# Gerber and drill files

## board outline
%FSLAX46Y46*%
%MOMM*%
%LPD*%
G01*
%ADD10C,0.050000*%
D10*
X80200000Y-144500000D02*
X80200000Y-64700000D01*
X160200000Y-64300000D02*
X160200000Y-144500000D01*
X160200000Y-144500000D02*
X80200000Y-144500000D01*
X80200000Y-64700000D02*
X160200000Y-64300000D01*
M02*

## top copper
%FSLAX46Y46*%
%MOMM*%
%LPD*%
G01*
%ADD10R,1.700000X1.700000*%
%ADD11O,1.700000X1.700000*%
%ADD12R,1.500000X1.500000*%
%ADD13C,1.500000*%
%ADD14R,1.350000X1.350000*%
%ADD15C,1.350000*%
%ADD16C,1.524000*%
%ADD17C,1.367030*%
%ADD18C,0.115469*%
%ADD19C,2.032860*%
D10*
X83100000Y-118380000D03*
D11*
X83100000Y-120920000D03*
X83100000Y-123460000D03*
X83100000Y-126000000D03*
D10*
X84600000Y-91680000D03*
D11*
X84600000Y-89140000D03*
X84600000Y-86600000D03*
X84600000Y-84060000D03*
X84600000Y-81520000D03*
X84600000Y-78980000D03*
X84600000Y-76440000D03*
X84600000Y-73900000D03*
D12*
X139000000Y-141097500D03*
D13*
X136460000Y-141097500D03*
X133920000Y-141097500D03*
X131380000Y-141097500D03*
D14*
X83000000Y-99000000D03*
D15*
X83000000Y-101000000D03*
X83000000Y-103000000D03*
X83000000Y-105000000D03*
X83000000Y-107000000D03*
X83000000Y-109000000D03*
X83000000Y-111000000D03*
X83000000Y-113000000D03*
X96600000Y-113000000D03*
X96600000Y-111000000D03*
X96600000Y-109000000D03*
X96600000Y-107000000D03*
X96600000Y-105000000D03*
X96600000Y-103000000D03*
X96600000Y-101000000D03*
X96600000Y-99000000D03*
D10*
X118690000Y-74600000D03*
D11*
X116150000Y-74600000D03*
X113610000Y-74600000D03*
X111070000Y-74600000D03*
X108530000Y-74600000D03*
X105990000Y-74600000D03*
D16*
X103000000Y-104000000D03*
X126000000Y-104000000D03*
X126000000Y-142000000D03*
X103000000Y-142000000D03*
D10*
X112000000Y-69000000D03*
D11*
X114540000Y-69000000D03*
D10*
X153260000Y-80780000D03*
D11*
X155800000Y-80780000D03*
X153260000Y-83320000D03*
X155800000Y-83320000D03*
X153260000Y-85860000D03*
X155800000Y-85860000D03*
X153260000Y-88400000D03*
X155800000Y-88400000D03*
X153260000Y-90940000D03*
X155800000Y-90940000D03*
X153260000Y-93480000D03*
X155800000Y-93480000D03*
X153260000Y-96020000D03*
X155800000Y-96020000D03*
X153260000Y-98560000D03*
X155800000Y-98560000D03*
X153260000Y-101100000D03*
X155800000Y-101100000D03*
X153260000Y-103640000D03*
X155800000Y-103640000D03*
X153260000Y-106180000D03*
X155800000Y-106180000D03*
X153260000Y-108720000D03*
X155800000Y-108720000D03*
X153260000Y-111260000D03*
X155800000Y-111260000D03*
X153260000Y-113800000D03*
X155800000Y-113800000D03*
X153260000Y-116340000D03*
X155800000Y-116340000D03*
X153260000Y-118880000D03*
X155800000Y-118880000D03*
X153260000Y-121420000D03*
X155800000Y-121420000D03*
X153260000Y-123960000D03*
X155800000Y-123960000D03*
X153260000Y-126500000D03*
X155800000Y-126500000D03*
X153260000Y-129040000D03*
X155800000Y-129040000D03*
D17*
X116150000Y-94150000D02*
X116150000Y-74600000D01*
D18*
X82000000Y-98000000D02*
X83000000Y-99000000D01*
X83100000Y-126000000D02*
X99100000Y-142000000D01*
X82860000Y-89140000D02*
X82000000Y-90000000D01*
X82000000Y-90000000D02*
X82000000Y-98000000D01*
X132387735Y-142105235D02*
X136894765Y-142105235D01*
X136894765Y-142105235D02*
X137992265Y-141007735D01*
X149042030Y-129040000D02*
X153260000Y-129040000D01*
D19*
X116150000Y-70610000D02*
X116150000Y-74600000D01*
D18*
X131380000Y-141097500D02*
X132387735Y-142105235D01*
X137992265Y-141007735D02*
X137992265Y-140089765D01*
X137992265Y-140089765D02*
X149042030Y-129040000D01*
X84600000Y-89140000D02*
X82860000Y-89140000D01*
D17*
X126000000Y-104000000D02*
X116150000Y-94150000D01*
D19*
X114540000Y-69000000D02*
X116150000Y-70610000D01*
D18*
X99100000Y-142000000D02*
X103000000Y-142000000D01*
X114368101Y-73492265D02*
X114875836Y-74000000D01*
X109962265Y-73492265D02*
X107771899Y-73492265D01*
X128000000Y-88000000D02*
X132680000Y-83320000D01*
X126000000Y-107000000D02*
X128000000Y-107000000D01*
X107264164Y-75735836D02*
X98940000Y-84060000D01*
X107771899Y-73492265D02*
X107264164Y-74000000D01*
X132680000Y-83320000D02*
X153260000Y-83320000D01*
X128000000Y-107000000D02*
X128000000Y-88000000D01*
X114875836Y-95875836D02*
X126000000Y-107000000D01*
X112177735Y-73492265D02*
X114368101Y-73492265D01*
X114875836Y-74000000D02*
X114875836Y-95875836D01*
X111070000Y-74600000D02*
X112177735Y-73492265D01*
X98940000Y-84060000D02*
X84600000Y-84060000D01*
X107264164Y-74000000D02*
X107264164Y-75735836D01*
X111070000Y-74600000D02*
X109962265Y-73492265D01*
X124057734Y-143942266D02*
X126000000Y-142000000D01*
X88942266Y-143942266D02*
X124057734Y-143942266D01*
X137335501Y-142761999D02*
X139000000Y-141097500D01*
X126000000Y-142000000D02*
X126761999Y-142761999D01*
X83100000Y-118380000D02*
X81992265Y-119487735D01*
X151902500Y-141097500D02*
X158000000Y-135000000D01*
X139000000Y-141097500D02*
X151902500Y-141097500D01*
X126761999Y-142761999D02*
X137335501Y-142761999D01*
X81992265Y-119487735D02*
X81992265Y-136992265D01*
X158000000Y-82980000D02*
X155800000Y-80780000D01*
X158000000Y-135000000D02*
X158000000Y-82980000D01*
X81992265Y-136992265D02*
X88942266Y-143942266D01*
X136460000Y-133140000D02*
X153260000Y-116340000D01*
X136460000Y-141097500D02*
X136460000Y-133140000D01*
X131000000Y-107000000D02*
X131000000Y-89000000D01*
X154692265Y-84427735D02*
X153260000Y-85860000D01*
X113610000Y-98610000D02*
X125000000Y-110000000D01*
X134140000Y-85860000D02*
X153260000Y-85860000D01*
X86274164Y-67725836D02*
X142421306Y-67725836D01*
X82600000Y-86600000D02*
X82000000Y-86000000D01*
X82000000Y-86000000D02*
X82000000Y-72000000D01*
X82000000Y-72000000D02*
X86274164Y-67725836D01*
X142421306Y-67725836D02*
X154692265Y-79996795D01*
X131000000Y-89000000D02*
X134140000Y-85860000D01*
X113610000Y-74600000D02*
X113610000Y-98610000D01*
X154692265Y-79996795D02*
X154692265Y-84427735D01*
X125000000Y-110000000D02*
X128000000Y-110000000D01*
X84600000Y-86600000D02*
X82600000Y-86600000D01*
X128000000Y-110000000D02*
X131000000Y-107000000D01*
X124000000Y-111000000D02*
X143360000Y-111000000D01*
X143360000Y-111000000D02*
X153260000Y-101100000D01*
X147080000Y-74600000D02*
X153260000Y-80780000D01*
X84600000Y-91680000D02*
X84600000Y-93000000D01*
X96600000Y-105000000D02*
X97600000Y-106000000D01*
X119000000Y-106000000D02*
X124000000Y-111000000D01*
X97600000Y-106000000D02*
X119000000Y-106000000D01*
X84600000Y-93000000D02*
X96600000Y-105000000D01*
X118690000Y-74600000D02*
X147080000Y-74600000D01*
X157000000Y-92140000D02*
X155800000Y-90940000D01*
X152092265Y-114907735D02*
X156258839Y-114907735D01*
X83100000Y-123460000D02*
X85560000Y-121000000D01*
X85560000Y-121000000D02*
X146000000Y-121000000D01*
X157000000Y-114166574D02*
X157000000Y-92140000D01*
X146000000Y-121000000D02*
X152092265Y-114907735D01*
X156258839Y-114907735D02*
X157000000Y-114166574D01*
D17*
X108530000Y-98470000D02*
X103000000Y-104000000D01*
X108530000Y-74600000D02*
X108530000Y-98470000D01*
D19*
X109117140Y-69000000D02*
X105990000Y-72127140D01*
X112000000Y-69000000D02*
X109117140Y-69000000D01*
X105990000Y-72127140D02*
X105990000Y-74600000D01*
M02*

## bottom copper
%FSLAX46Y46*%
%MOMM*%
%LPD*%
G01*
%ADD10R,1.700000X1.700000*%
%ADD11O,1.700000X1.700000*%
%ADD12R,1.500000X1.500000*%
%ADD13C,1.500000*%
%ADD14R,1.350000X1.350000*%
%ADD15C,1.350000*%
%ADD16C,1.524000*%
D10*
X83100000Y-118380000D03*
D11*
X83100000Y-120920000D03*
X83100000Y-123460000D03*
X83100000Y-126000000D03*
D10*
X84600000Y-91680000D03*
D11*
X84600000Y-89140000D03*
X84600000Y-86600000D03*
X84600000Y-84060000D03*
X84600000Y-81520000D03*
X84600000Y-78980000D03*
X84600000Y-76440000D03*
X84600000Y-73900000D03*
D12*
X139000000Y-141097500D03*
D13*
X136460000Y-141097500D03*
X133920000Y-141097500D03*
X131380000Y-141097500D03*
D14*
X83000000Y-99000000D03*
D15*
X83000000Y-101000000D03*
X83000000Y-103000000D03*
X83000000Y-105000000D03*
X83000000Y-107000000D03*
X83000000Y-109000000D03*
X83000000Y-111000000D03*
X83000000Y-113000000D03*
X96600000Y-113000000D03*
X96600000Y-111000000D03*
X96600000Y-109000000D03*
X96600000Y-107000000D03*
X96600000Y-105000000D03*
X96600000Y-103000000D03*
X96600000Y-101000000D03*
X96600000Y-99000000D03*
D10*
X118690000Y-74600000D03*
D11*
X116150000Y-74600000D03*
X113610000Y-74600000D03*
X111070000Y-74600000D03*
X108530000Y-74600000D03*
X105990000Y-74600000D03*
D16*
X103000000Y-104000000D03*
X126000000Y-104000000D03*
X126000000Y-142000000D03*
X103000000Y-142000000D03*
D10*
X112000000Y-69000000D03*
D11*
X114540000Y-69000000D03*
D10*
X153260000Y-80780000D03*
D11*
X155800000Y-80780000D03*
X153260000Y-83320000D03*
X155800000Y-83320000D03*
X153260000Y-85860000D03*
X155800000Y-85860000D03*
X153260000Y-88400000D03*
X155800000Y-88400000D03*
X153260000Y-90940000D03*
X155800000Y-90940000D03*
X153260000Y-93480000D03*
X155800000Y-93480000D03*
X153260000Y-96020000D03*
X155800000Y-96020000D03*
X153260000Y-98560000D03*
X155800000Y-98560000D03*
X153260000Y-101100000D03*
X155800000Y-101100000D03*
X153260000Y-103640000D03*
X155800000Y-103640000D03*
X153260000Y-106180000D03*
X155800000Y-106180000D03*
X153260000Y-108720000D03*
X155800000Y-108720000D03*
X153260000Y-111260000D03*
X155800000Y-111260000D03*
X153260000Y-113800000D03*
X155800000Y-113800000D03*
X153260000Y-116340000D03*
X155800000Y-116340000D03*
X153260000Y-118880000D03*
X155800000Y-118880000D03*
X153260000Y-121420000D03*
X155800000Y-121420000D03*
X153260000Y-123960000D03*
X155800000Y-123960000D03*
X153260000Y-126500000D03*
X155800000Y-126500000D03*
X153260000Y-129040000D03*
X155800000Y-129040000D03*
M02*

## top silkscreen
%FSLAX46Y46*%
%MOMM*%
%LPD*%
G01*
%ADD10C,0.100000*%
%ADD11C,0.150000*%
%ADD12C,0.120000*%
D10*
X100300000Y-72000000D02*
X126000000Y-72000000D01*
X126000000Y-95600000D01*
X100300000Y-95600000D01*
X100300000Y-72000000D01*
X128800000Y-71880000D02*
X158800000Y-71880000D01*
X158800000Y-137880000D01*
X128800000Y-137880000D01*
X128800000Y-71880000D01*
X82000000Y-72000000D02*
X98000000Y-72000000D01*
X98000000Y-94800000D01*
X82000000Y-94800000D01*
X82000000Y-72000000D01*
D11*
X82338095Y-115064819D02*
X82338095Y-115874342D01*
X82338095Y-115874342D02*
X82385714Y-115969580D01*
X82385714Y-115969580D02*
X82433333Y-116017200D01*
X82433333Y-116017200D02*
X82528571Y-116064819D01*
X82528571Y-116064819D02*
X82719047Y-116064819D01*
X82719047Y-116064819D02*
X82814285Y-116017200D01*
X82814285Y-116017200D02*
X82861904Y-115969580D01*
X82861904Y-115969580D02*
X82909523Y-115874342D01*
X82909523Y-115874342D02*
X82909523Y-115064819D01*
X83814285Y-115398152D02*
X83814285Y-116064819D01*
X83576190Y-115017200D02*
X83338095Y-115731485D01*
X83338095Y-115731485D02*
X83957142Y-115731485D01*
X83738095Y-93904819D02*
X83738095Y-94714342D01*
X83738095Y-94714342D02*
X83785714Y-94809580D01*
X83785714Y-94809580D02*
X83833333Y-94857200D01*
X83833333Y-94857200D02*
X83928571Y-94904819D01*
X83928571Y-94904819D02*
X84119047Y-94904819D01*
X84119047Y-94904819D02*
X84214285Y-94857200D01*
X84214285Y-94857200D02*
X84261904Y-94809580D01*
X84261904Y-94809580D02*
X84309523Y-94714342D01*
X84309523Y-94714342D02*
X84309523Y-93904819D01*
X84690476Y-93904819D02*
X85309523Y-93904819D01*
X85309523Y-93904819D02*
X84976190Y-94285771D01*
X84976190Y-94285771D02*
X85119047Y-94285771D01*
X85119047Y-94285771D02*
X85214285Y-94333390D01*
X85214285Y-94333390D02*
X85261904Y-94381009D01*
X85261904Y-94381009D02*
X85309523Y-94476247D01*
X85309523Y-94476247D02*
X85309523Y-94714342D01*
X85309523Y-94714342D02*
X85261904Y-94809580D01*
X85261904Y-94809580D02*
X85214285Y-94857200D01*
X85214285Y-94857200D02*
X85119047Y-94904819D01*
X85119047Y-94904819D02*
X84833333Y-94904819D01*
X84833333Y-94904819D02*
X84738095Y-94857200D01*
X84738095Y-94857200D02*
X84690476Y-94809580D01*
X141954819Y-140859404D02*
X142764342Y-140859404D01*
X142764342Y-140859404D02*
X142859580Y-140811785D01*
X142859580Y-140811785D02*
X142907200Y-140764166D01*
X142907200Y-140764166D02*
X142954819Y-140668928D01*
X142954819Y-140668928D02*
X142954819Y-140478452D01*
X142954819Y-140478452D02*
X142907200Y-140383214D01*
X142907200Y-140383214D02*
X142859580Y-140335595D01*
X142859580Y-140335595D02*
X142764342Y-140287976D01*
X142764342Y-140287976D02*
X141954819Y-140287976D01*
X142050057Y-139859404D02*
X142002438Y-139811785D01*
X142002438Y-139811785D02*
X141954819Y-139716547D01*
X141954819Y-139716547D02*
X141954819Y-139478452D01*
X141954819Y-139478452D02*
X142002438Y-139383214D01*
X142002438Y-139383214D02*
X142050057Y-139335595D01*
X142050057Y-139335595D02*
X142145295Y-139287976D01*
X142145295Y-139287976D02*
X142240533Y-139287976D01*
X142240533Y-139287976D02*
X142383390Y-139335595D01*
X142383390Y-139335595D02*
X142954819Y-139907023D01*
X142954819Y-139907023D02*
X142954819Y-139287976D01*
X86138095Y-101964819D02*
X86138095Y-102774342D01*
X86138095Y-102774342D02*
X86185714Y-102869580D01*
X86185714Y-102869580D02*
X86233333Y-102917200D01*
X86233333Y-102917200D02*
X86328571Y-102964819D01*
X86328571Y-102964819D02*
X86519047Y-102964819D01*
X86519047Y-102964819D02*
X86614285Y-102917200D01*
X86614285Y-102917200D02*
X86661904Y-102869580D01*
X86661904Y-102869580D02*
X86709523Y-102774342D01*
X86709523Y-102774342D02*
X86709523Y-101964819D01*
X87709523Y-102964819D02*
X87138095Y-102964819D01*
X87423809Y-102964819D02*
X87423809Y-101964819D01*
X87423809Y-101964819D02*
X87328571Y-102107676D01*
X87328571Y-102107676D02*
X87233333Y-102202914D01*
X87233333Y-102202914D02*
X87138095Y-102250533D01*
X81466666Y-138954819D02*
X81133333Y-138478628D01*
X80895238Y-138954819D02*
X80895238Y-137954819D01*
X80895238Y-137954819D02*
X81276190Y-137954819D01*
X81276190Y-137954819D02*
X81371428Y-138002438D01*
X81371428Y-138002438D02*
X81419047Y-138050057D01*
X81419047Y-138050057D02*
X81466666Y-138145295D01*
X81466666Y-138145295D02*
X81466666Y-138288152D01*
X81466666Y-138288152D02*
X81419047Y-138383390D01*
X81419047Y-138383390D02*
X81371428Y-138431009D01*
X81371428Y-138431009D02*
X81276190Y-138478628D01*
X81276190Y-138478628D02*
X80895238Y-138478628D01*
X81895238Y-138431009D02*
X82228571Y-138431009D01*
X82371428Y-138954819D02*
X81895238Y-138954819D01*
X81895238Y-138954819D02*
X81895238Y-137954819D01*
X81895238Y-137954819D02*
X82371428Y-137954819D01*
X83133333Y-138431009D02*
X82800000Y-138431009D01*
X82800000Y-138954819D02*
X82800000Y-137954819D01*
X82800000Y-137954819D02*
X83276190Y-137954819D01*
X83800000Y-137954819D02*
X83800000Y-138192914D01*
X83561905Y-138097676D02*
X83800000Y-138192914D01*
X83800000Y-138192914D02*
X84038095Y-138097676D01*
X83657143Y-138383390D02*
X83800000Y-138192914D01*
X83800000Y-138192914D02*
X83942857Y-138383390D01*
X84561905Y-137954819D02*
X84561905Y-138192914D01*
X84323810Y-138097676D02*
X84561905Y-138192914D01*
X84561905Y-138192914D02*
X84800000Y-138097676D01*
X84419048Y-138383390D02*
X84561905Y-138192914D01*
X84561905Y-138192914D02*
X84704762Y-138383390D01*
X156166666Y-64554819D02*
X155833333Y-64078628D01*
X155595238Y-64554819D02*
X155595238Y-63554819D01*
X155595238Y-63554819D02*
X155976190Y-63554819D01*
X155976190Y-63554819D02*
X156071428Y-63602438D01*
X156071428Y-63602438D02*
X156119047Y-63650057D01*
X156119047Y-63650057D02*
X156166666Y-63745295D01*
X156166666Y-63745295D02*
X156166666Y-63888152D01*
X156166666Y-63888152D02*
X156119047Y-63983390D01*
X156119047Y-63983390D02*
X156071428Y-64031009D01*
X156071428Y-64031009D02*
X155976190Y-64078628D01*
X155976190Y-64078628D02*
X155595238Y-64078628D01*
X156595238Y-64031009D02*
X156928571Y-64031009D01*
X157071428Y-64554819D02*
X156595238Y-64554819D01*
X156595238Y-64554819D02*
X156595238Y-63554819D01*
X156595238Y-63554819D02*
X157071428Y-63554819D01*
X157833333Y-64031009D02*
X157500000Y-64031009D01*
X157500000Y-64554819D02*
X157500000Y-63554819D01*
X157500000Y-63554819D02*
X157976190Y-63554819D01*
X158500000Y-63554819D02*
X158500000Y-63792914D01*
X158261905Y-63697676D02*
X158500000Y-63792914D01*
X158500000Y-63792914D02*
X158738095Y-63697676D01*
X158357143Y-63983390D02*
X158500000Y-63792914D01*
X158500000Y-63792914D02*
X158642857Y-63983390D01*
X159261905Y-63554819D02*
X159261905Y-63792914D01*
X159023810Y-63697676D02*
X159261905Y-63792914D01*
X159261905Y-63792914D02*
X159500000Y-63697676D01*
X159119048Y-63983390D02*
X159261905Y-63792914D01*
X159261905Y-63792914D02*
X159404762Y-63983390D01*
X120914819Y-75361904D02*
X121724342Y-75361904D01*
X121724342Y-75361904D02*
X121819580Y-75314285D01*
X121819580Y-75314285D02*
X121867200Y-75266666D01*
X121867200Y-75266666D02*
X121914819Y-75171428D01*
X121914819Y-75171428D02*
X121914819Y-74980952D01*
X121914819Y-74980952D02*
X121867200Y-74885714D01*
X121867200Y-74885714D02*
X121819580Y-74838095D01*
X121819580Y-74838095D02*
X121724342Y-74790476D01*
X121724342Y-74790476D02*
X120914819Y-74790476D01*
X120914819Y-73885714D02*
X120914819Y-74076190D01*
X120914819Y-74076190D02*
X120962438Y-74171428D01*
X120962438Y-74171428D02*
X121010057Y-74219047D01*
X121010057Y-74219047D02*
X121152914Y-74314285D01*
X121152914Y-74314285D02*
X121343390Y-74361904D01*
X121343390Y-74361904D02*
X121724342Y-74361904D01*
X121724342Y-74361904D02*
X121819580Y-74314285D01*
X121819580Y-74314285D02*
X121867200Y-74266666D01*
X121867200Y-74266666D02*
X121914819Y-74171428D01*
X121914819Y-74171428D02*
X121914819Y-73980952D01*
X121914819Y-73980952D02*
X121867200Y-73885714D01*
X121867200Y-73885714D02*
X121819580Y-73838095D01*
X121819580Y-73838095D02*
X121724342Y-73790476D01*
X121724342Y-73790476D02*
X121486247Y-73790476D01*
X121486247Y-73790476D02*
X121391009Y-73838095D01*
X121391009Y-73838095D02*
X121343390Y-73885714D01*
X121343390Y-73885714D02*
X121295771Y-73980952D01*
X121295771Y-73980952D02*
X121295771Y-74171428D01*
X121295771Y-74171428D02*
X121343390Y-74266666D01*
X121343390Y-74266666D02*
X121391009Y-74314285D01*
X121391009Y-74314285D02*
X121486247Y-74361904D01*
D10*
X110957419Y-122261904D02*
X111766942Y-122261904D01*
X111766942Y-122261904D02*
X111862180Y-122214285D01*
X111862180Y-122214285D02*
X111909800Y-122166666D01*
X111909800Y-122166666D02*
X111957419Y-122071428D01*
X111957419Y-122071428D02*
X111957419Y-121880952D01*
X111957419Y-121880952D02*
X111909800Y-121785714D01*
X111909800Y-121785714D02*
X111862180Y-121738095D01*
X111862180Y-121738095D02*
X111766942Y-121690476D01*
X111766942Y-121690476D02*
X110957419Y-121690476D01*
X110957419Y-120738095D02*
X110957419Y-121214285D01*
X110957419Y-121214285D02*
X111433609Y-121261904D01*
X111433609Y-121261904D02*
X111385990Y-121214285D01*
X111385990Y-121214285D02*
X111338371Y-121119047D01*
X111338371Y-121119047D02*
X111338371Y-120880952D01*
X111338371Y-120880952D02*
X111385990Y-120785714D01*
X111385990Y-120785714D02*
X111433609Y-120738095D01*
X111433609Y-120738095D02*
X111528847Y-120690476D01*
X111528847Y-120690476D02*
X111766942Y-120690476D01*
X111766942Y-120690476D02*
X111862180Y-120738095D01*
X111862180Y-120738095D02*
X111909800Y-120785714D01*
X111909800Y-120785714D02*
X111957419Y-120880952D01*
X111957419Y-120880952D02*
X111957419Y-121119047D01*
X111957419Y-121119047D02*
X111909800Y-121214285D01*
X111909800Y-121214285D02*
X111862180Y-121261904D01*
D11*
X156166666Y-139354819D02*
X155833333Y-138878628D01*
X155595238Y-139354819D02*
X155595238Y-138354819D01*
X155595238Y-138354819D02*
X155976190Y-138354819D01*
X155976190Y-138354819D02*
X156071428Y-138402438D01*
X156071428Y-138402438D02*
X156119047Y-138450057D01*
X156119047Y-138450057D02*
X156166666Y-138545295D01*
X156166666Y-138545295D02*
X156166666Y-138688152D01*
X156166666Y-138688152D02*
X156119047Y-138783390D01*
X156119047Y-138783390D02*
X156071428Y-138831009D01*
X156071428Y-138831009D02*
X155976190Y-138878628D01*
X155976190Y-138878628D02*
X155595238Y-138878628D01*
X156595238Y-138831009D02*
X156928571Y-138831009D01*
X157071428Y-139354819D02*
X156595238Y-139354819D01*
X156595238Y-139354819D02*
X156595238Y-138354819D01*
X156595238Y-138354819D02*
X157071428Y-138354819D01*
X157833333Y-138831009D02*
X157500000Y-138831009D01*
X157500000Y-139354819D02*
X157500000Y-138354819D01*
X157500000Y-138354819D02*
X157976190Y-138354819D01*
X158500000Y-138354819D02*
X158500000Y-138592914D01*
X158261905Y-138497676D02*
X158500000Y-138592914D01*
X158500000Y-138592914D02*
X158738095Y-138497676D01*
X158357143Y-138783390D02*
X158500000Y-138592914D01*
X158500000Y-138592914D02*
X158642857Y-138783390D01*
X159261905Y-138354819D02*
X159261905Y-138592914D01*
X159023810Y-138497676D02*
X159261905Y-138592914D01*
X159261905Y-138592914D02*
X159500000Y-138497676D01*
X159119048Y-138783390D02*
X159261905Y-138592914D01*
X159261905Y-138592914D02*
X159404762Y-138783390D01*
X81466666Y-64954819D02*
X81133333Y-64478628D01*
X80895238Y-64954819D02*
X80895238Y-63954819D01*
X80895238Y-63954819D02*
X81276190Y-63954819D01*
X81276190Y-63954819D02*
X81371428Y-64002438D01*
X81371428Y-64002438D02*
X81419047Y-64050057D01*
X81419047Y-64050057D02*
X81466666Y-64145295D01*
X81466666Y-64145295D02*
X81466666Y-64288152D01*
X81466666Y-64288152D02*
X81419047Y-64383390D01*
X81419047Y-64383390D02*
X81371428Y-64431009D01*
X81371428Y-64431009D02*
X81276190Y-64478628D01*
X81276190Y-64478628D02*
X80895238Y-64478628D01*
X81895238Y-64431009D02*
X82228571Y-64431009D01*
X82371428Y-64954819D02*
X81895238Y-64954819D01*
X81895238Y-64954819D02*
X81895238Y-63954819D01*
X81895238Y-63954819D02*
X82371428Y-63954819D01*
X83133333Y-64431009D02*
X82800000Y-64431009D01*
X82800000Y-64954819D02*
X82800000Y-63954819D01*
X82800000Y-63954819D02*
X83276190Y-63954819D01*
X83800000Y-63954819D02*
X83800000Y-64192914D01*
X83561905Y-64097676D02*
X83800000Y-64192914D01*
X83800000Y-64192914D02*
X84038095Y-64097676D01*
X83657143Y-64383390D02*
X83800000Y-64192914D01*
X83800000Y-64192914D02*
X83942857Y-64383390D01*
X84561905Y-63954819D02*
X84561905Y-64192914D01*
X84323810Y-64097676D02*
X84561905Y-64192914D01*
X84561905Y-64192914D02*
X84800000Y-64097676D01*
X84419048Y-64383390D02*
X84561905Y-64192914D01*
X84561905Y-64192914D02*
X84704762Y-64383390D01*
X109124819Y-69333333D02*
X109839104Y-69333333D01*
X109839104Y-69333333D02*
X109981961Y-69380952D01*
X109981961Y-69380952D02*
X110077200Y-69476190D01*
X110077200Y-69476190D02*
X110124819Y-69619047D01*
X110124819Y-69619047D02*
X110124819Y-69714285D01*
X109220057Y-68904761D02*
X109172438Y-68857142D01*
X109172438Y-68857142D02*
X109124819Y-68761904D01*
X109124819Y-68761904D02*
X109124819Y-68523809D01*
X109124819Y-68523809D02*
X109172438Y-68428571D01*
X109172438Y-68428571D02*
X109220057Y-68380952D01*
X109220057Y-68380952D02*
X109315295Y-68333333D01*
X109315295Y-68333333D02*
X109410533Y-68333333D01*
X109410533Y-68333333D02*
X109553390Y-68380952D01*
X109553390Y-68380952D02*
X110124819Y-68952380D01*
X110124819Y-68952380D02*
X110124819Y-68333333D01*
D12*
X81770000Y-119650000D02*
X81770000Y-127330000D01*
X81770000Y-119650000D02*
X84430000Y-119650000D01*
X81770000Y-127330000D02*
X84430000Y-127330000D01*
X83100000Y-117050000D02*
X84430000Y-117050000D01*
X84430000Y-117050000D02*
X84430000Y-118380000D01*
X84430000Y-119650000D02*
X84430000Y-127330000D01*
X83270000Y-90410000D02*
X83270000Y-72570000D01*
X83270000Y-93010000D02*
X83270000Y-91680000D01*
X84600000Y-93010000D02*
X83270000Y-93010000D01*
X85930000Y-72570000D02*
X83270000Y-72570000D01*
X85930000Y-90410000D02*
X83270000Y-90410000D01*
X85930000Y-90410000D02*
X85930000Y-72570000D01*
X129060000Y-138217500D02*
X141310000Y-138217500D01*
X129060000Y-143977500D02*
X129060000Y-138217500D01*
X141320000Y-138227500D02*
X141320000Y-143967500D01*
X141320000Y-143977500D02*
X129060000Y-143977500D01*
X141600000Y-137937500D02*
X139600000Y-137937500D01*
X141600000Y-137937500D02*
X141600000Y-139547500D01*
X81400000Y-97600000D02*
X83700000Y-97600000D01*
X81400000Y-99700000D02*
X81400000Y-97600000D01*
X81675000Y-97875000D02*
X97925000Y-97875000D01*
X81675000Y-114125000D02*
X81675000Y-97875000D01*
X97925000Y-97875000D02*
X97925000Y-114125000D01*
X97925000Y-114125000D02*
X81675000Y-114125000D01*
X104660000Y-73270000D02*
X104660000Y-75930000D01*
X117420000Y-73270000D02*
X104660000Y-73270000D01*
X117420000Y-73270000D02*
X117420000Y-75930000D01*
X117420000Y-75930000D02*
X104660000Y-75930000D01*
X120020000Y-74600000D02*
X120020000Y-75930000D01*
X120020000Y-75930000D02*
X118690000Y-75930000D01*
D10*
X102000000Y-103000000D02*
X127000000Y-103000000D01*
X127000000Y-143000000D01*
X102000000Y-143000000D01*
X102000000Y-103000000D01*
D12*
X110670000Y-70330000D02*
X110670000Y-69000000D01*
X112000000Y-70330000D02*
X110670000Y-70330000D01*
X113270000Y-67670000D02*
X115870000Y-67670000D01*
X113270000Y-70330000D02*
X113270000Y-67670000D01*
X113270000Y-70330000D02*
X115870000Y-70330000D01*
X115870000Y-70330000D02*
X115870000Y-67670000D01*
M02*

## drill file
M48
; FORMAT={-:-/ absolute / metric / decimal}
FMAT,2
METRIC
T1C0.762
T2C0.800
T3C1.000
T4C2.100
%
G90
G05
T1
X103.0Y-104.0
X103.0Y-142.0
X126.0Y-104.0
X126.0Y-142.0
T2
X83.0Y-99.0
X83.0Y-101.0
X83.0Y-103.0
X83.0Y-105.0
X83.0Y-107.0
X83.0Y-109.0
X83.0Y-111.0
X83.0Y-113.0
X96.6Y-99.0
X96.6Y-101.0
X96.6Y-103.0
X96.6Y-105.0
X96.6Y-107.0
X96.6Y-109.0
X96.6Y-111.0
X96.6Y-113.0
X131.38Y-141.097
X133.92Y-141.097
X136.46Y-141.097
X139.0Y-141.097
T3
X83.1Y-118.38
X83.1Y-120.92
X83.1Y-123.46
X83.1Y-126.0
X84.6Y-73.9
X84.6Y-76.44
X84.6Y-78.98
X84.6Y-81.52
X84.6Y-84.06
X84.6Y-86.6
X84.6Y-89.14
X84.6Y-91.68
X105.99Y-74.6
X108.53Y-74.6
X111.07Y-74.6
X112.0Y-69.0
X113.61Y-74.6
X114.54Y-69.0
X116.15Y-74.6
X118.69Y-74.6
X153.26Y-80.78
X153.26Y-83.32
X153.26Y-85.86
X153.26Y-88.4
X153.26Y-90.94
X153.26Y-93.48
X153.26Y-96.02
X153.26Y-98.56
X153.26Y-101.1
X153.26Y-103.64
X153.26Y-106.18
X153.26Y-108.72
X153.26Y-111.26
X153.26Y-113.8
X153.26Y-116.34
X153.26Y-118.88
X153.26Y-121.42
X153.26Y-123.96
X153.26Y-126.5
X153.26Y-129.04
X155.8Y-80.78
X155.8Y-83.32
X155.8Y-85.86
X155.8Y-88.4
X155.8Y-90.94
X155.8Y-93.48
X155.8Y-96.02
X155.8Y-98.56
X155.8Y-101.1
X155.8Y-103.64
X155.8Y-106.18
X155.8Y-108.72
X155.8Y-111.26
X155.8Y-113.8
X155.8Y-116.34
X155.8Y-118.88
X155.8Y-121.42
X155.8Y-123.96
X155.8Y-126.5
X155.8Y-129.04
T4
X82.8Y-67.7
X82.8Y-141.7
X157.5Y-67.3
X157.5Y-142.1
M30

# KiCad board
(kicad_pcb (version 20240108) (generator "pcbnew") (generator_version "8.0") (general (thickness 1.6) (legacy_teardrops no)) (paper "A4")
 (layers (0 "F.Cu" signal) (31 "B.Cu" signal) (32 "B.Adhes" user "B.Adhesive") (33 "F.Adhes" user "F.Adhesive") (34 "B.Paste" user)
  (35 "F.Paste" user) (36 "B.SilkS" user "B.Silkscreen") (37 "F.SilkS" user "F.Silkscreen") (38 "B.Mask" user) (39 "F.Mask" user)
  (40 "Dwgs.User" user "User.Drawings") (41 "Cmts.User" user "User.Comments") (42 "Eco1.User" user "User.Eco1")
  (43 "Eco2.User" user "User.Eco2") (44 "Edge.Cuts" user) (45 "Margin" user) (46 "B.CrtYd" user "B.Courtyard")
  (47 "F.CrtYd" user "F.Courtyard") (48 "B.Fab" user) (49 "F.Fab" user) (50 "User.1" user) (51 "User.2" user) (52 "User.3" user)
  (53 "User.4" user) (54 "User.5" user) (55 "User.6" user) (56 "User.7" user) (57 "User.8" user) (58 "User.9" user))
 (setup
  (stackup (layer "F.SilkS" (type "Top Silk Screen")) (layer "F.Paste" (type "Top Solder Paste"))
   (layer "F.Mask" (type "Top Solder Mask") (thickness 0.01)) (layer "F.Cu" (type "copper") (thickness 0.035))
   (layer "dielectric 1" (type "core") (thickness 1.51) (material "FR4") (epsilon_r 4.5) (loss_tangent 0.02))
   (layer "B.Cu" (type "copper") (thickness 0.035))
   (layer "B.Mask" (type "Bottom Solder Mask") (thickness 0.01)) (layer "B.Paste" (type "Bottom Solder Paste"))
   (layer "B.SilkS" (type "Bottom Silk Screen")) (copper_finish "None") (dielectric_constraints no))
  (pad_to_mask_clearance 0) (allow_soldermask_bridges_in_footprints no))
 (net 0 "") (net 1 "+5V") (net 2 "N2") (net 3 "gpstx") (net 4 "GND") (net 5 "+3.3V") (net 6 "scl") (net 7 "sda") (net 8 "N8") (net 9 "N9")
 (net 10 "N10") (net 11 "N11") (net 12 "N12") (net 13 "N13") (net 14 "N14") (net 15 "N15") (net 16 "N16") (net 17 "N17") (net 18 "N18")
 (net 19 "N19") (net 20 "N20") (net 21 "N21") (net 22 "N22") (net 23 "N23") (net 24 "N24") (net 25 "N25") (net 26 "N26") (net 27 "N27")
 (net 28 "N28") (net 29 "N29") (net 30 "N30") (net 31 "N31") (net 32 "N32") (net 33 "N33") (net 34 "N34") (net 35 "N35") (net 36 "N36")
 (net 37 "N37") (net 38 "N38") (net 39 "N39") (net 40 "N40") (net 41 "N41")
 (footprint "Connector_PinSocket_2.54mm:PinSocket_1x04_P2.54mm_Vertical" (layer "F.Cu") (at 83.1 118.38)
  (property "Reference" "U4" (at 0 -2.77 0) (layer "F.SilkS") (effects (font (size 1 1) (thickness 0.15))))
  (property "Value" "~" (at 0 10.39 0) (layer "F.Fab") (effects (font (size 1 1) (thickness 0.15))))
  (fp_line (start -1.33 1.27) (end -1.33 8.95) (stroke (width 0.12) (type solid)) (layer "F.SilkS"))
  (fp_line (start -1.33 1.27) (end 1.33 1.27) (stroke (width 0.12) (type solid)) (layer "F.SilkS"))
  (fp_line (start -1.33 8.95) (end 1.33 8.95) (stroke (width 0.12) (type solid)) (layer "F.SilkS"))
  (fp_line (start 0 -1.33) (end 1.33 -1.33) (stroke (width 0.12) (type solid)) (layer "F.SilkS"))
  (fp_line (start 1.33 -1.33) (end 1.33 0) (stroke (width 0.12) (type solid)) (layer "F.SilkS"))
  (fp_line (start 1.33 1.27) (end 1.33 8.95) (stroke (width 0.12) (type solid)) (layer "F.SilkS"))
  (pad "1" thru_hole rect (at 0 0) (size 1.7 1.7) (drill 1) (layers "*.Cu" "*.Mask") (remove_unused_layers no) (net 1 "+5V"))
  (pad "2" thru_hole oval (at 0 2.54) (size 1.7 1.7) (drill 1) (layers "*.Cu" "*.Mask") (remove_unused_layers no) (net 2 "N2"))
  (pad "3" thru_hole oval (at 0 5.08) (size 1.7 1.7) (drill 1) (layers "*.Cu" "*.Mask") (remove_unused_layers no) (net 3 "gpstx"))
  (pad "4" thru_hole oval (at 0 7.62) (size 1.7 1.7) (drill 1) (layers "*.Cu" "*.Mask") (remove_unused_layers no) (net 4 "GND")))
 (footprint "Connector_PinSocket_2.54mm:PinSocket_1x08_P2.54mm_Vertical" (layer "F.Cu") (at 84.6 91.68 180)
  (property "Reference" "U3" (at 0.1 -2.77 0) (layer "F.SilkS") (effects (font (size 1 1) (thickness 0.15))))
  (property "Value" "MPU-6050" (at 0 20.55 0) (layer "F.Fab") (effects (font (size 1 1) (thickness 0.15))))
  (fp_line (start 1.33 1.27) (end 1.33 19.11) (stroke (width 0.12) (type solid)) (layer "F.SilkS"))
  (fp_line (start 1.33 -1.33) (end 1.33 0) (stroke (width 0.12) (type solid)) (layer "F.SilkS"))
  (fp_line (start 0 -1.33) (end 1.33 -1.33) (stroke (width 0.12) (type solid)) (layer "F.SilkS"))
  (fp_line (start -1.33 19.11) (end 1.33 19.11) (stroke (width 0.12) (type solid)) (layer "F.SilkS"))
  (fp_line (start -1.33 1.27) (end 1.33 1.27) (stroke (width 0.12) (type solid)) (layer "F.SilkS"))
  (fp_line (start -1.33 1.27) (end -1.33 19.11) (stroke (width 0.12) (type solid)) (layer "F.SilkS"))
  (pad "1" thru_hole rect (at 0 0 180) (size 1.7 1.7) (drill 1) (layers "*.Cu" "*.Mask") (remove_unused_layers no) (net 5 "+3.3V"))
  (pad "2" thru_hole oval (at 0 2.54 180) (size 1.7 1.7) (drill 1) (layers "*.Cu" "*.Mask") (remove_unused_layers no) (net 4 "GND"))
  (pad "3" thru_hole oval (at 0 5.08 180) (size 1.7 1.7) (drill 1) (layers "*.Cu" "*.Mask") (remove_unused_layers no) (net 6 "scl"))
  (pad "4" thru_hole oval (at 0 7.62 180) (size 1.7 1.7) (drill 1) (layers "*.Cu" "*.Mask") (remove_unused_layers no) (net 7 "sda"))
  (pad "5" thru_hole oval (at 0 10.16 180) (size 1.7 1.7) (drill 1) (layers "*.Cu" "*.Mask") (remove_unused_layers no) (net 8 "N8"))
  (pad "6" thru_hole oval (at 0 12.7 180) (size 1.7 1.7) (drill 1) (layers "*.Cu" "*.Mask") (remove_unused_layers no) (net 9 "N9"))
  (pad "7" thru_hole oval (at 0 15.24 180) (size 1.7 1.7) (drill 1) (layers "*.Cu" "*.Mask") (remove_unused_layers no) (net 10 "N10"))
  (pad "8" thru_hole oval (at 0 17.78 180) (size 1.7 1.7) (drill 1) (layers "*.Cu" "*.Mask") (remove_unused_layers no) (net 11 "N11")))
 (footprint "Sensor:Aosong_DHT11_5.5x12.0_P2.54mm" (layer "F.Cu") (at 139 141.0975 -90)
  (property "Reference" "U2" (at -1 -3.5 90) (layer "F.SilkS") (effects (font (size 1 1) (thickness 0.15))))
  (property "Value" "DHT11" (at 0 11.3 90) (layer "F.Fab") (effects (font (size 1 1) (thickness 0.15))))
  (fp_line (start -2.88 9.94) (end -2.88 -2.31) (stroke (width 0.12) (type solid)) (layer "F.SilkS"))
  (fp_line (start 2.88 9.94) (end -2.88 9.94) (stroke (width 0.12) (type solid)) (layer "F.SilkS"))
  (fp_line (start -2.87 -2.32) (end 2.87 -2.32) (stroke (width 0.12) (type solid)) (layer "F.SilkS"))
  (fp_line (start 2.88 -2.32) (end 2.88 9.94) (stroke (width 0.12) (type solid)) (layer "F.SilkS"))
  (fp_line (start -3.16 -2.6) (end -3.16 -0.6) (stroke (width 0.12) (type solid)) (layer "F.SilkS"))
  (fp_line (start -3.16 -2.6) (end -1.55 -2.6) (stroke (width 0.12) (type solid)) (layer "F.SilkS"))
  (pad "1" thru_hole rect (at 0 0 270) (size 1.5 1.5) (drill 0.8) (layers "*.Cu" "*.Mask") (remove_unused_layers no) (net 1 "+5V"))
  (pad "2" thru_hole circle (at 0 2.54 270) (size 1.5 1.5) (drill 0.8) (layers "*.Cu" "*.Mask") (remove_unused_layers no) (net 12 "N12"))
  (pad "3" thru_hole circle (at 0 5.08 270) (size 1.5 1.5) (drill 0.8) (layers "*.Cu" "*.Mask") (remove_unused_layers no) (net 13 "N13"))
  (pad "4" thru_hole circle (at 0 7.62 270) (size 1.5 1.5) (drill 0.8) (layers "*.Cu" "*.Mask") (remove_unused_layers no) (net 4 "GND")))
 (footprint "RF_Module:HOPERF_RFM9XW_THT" (layer "F.Cu") (at 83 99)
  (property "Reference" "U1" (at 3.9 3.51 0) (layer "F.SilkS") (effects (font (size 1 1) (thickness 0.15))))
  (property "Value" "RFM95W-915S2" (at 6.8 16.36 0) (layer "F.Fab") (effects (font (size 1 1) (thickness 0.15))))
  (fp_line (start -1.6 -1.4) (end 0.7 -1.4) (stroke (width 0.12) (type solid)) (layer "F.SilkS"))
  (fp_line (start -1.6 0.7) (end -1.6 -1.4) (stroke (width 0.12) (type solid)) (layer "F.SilkS"))
  (fp_line (start -1.325 -1.125) (end 14.925 -1.125) (stroke (width 0.12) (type solid)) (layer "F.SilkS"))
  (fp_line (start -1.325 15.125) (end -1.325 -1.125) (stroke (width 0.12) (type solid)) (layer "F.SilkS"))
  (fp_line (start 14.925 -1.125) (end 14.925 15.125) (stroke (width 0.12) (type solid)) (layer "F.SilkS"))
  (fp_line (start 14.925 15.125) (end -1.325 15.125) (stroke (width 0.12) (type solid)) (layer "F.SilkS"))
  (pad "1" thru_hole rect (at 0 0) (size 1.35 1.35) (drill 0.8) (layers "*.Cu" "*.Mask") (remove_unused_layers no) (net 4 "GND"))
  (pad "2" thru_hole circle (at 0 2) (size 1.35 1.35) (drill 0.8) (layers "*.Cu" "*.Mask") (remove_unused_layers no) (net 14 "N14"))
  (pad "3" thru_hole circle (at 0 4) (size 1.35 1.35) (drill 0.8) (layers "*.Cu" "*.Mask") (remove_unused_layers no) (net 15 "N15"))
  (pad "4" thru_hole circle (at 0 6) (size 1.35 1.35) (drill 0.8) (layers "*.Cu" "*.Mask") (remove_unused_layers no) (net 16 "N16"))
  (pad "5" thru_hole circle (at 0 8) (size 1.35 1.35) (drill 0.8) (layers "*.Cu" "*.Mask") (remove_unused_layers no) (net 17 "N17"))
  (pad "6" thru_hole circle (at 0 10) (size 1.35 1.35) (drill 0.8) (layers "*.Cu" "*.Mask") (remove_unused_layers no) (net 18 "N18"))
  (pad "7" thru_hole circle (at 0 12) (size 1.35 1.35) (drill 0.8) (layers "*.Cu" "*.Mask") (remove_unused_layers no) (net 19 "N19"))
  (pad "8" thru_hole circle (at 0 14) (size 1.35 1.35) (drill 0.8) (layers "*.Cu" "*.Mask") (remove_unused_layers no) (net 4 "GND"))
  (pad "9" thru_hole circle (at 13.6 14) (size 1.35 1.35) (drill 0.8) (layers "*.Cu" "*.Mask") (remove_unused_layers no) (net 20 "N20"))
  (pad "10" thru_hole circle (at 13.6 12) (size 1.35 1.35) (drill 0.8) (layers "*.Cu" "*.Mask") (remove_unused_layers no) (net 4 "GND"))
  (pad "11" thru_hole circle (at 13.6 10) (size 1.35 1.35) (drill 0.8) (layers "*.Cu" "*.Mask") (remove_unused_layers no) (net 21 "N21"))
  (pad "12" thru_hole circle (at 13.6 8) (size 1.35 1.35) (drill 0.8) (layers "*.Cu" "*.Mask") (remove_unused_layers no) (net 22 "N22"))
  (pad "13" thru_hole circle (at 13.6 6) (size 1.35 1.35) (drill 0.8) (layers "*.Cu" "*.Mask") (remove_unused_layers no) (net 5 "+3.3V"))
  (pad "14" thru_hole circle (at 13.6 4) (size 1.35 1.35) (drill 0.8) (layers "*.Cu" "*.Mask") (remove_unused_layers no) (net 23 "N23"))
  (pad "15" thru_hole circle (at 13.6 2) (size 1.35 1.35) (drill 0.8) (layers "*.Cu" "*.Mask") (remove_unused_layers no) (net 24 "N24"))
  (pad "16" thru_hole circle (at 13.6 0) (size 1.35 1.35) (drill 0.8) (layers "*.Cu" "*.Mask") (remove_unused_layers no) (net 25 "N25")))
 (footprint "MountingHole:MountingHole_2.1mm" (layer "F.Cu") (at 82.8 141.7)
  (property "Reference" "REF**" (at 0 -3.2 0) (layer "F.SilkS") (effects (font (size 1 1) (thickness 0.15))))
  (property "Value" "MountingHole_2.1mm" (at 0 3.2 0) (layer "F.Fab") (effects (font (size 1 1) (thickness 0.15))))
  (pad "" np_thru_hole circle (at 0 0) (size 2.1 2.1) (drill 2.1) (layers "*.Cu" "*.Mask")))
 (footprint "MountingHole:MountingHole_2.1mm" (layer "F.Cu") (at 157.5 67.3)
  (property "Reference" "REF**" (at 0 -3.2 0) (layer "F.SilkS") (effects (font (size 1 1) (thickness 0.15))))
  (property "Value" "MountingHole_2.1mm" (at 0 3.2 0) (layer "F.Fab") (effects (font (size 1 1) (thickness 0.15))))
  (pad "" np_thru_hole circle (at 0 0) (size 2.1 2.1) (drill 2.1) (layers "*.Cu" "*.Mask")))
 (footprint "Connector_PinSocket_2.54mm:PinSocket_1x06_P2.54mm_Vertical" (layer "F.Cu") (at 118.69 74.6 -90)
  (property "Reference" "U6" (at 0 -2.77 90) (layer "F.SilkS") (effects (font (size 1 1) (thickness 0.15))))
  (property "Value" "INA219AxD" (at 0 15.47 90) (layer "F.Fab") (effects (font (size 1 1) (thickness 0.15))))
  (fp_line (start -1.33 14.03) (end 1.33 14.03) (stroke (width 0.12) (type solid)) (layer "F.SilkS"))
  (fp_line (start -1.33 1.27) (end -1.33 14.03) (stroke (width 0.12) (type solid)) (layer "F.SilkS"))
  (fp_line (start -1.33 1.27) (end 1.33 1.27) (stroke (width 0.12) (type solid)) (layer "F.SilkS"))
  (fp_line (start 1.33 1.27) (end 1.33 14.03) (stroke (width 0.12) (type solid)) (layer "F.SilkS"))
  (fp_line (start 0 -1.33) (end 1.33 -1.33) (stroke (width 0.12) (type solid)) (layer "F.SilkS"))
  (fp_line (start 1.33 -1.33) (end 1.33 0) (stroke (width 0.12) (type solid)) (layer "F.SilkS"))
  (pad "1" thru_hole rect (at 0 0 270) (size 1.7 1.7) (drill 1) (layers "*.Cu" "*.Mask") (remove_unused_layers no) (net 5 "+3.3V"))
  (pad "2" thru_hole oval (at 0 2.54 270) (size 1.7 1.7) (drill 1) (layers "*.Cu" "*.Mask") (remove_unused_layers no) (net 4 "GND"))
  (pad "3" thru_hole oval (at 0 5.08 270) (size 1.7 1.7) (drill 1) (layers "*.Cu" "*.Mask") (remove_unused_layers no) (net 6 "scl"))
  (pad "4" thru_hole oval (at 0 7.62 270) (size 1.7 1.7) (drill 1) (layers "*.Cu" "*.Mask") (remove_unused_layers no) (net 7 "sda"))
  (pad "5" thru_hole oval (at 0 10.16 270) (size 1.7 1.7) (drill 1) (layers "*.Cu" "*.Mask") (remove_unused_layers no) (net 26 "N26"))
  (pad "6" thru_hole oval (at 0 12.7 270) (size 1.7 1.7) (drill 1) (layers "*.Cu" "*.Mask") (remove_unused_layers no) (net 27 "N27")))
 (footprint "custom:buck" (layer "F.Cu") (at 112.5 121.5 90)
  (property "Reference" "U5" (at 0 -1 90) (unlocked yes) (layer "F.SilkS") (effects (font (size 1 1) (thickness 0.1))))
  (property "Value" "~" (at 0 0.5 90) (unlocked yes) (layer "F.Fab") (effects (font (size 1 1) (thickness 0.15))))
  (fp_rect (start -21.5 -10.5) (end 18.5 14.5) (stroke (width 0.1) (type default)) (fill none) (layer "F.SilkS"))
  (pad "1" thru_hole circle (at 17.5 -9.5 90) (size 1.524 1.524) (drill 0.762) (layers "*.Cu" "*.Mask") (remove_unused_layers no)
   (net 26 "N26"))
  (pad "2" thru_hole circle (at 17.5 13.5 90) (size 1.524 1.524) (drill 0.762) (layers "*.Cu" "*.Mask") (remove_unused_layers no)
   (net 4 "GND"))
  (pad "3" thru_hole circle (at -20.5 13.5 90) (size 1.524 1.524) (drill 0.762) (layers "*.Cu" "*.Mask") (remove_unused_layers no)
   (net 1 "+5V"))
  (pad "4" thru_hole circle (at -20.5 -9.5 90) (size 1.524 1.524) (drill 0.762) (layers "*.Cu" "*.Mask") (remove_unused_layers no)
   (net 4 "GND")))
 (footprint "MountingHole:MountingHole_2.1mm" (layer "F.Cu") (at 157.5 142.1)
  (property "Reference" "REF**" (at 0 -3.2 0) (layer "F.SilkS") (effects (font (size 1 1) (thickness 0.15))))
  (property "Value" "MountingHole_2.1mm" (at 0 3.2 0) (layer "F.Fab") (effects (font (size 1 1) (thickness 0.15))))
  (pad "" np_thru_hole circle (at 0 0) (size 2.1 2.1) (drill 2.1) (layers "*.Cu" "*.Mask")))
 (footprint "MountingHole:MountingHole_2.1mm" (layer "F.Cu") (at 82.8 67.7)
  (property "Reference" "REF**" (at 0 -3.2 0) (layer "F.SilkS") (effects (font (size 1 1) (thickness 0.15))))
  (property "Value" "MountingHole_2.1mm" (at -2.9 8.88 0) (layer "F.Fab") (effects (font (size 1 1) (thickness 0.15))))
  (pad "" np_thru_hole circle (at 0 0) (size 2.1 2.1) (drill 2.1) (layers "*.Cu" "*.Mask")))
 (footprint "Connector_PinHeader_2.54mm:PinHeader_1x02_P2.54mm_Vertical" (layer "F.Cu") (at 112 69 90)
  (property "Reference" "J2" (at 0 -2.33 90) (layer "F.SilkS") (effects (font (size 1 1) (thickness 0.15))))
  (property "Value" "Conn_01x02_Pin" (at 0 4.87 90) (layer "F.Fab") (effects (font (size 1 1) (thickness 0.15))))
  (fp_line (start -1.33 -1.33) (end 0 -1.33) (stroke (width 0.12) (type solid)) (layer "F.SilkS"))
  (fp_line (start -1.33 0) (end -1.33 -1.33) (stroke (width 0.12) (type solid)) (layer "F.SilkS"))
  (fp_line (start 1.33 1.27) (end 1.33 3.87) (stroke (width 0.12) (type solid)) (layer "F.SilkS"))
  (fp_line (start -1.33 1.27) (end 1.33 1.27) (stroke (width 0.12) (type solid)) (layer "F.SilkS"))
  (fp_line (start -1.33 1.27) (end -1.33 3.87) (stroke (width 0.12) (type solid)) (layer "F.SilkS"))
  (fp_line (start -1.33 3.87) (end 1.33 3.87) (stroke (width 0.12) (type solid)) (layer "F.SilkS"))
  (pad "1" thru_hole rect (at 0 0 90) (size 1.7 1.7) (drill 1) (layers "*.Cu" "*.Mask") (remove_unused_layers no) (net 27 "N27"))
  (pad "2" thru_hole oval (at 0 2.54 90) (size 1.7 1.7) (drill 1) (layers "*.Cu" "*.Mask") (remove_unused_layers no) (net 4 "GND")))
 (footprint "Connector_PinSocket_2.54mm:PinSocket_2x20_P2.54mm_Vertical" (layer "B.Cu") (at 153.26 80.78 180)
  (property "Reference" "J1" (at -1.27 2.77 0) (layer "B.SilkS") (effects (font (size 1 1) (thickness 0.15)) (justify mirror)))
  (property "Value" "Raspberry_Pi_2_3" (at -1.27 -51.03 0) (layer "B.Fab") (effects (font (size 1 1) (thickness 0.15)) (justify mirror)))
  (pad "1" thru_hole rect (at 0 0 180) (size 1.7 1.7) (drill 1) (layers "*.Cu" "*.Mask") (remove_unused_layers no) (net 5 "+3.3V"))
  (pad "2" thru_hole oval (at -2.54 0 180) (size 1.7 1.7) (drill 1) (layers "*.Cu" "*.Mask") (remove_unused_layers no) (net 1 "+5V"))
  (pad "3" thru_hole oval (at 0 -2.54 180) (size 1.7 1.7) (drill 1) (layers "*.Cu" "*.Mask") (remove_unused_layers no) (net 7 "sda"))
  (pad "4" thru_hole oval (at -2.54 -2.54 180) (size 1.7 1.7) (drill 1) (layers "*.Cu" "*.Mask") (remove_unused_layers no) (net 1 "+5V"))
  (pad "5" thru_hole oval (at 0 -5.08 180) (size 1.7 1.7) (drill 1) (layers "*.Cu" "*.Mask") (remove_unused_layers no) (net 6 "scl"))
  (pad "6" thru_hole oval (at -2.54 -5.08 180) (size 1.7 1.7) (drill 1) (layers "*.Cu" "*.Mask") (remove_unused_layers no) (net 4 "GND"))
  (pad "7" thru_hole oval (at 0 -7.62 180) (size 1.7 1.7) (drill 1) (layers "*.Cu" "*.Mask") (remove_unused_layers no) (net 23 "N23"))
  (pad "8" thru_hole oval (at -2.54 -7.62 180) (size 1.7 1.7) (drill 1) (layers "*.Cu" "*.Mask") (remove_unused_layers no) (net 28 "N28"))
  (pad "9" thru_hole oval (at 0 -10.16 180) (size 1.7 1.7) (drill 1) (layers "*.Cu" "*.Mask") (remove_unused_layers no) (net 4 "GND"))
  (pad "10" thru_hole oval (at -2.54 -10.16 180) (size 1.7 1.7) (drill 1) (layers "*.Cu" "*.Mask") (remove_unused_layers no) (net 3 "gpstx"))
  (pad "11" thru_hole oval (at 0 -12.7 180) (size 1.7 1.7) (drill 1) (layers "*.Cu" "*.Mask") (remove_unused_layers no) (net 24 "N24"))
  (pad "12" thru_hole oval (at -2.54 -12.7 180) (size 1.7 1.7) (drill 1) (layers "*.Cu" "*.Mask") (remove_unused_layers no) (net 25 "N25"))
  (pad "13" thru_hole oval (at 0 -15.24 180) (size 1.7 1.7) (drill 1) (layers "*.Cu" "*.Mask") (remove_unused_layers no) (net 21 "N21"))
  (pad "14" thru_hole oval (at -2.54 -15.24 180) (size 1.7 1.7) (drill 1) (layers "*.Cu" "*.Mask") (remove_unused_layers no) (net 4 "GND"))
  (pad "15" thru_hole oval (at 0 -17.78 180) (size 1.7 1.7) (drill 1) (layers "*.Cu" "*.Mask") (remove_unused_layers no) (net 18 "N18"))
  (pad "16" thru_hole oval (at -2.54 -17.78 180) (size 1.7 1.7) (drill 1) (layers "*.Cu" "*.Mask") (remove_unused_layers no) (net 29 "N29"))
  (pad "17" thru_hole oval (at 0 -20.32 180) (size 1.7 1.7) (drill 1) (layers "*.Cu" "*.Mask") (remove_unused_layers no) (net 5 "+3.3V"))
  (pad "18" thru_hole oval (at -2.54 -20.32 180) (size 1.7 1.7) (drill 1) (layers "*.Cu" "*.Mask") (remove_unused_layers no) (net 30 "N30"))
  (pad "19" thru_hole oval (at 0 -22.86 180) (size 1.7 1.7) (drill 1) (layers "*.Cu" "*.Mask") (remove_unused_layers no) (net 15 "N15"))
  (pad "20" thru_hole oval (at -2.54 -22.86 180) (size 1.7 1.7) (drill 1) (layers "*.Cu" "*.Mask") (remove_unused_layers no) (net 4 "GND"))
  (pad "21" thru_hole oval (at 0 -25.4 180) (size 1.7 1.7) (drill 1) (layers "*.Cu" "*.Mask") (remove_unused_layers no) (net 14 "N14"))
  (pad "22" thru_hole oval (at -2.54 -25.4 180) (size 1.7 1.7) (drill 1) (layers "*.Cu" "*.Mask") (remove_unused_layers no) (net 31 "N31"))
  (pad "23" thru_hole oval (at 0 -27.94 180) (size 1.7 1.7) (drill 1) (layers "*.Cu" "*.Mask") (remove_unused_layers no) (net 16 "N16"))
  (pad "24" thru_hole oval (at -2.54 -27.94 180) (size 1.7 1.7) (drill 1) (layers "*.Cu" "*.Mask") (remove_unused_layers no) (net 17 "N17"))
  (pad "25" thru_hole oval (at 0 -30.48 180) (size 1.7 1.7) (drill 1) (layers "*.Cu" "*.Mask") (remove_unused_layers no) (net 4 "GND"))
  (pad "26" thru_hole oval (at -2.54 -30.48 180) (size 1.7 1.7) (drill 1) (layers "*.Cu" "*.Mask") (remove_unused_layers no) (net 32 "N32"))
  (pad "27" thru_hole oval (at 0 -33.02 180) (size 1.7 1.7) (drill 1) (layers "*.Cu" "*.Mask") (remove_unused_layers no) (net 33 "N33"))
  (pad "28" thru_hole oval (at -2.54 -33.02 180) (size 1.7 1.7) (drill 1) (layers "*.Cu" "*.Mask") (remove_unused_layers no) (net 33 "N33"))
  (pad "29" thru_hole oval (at 0 -35.56 180) (size 1.7 1.7) (drill 1) (layers "*.Cu" "*.Mask") (remove_unused_layers no) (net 12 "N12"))
  (pad "30" thru_hole oval (at -2.54 -35.56 180) (size 1.7 1.7) (drill 1) (layers "*.Cu" "*.Mask") (remove_unused_layers no) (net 4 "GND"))
  (pad "31" thru_hole oval (at 0 -38.1 180) (size 1.7 1.7) (drill 1) (layers "*.Cu" "*.Mask") (remove_unused_layers no) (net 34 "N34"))
  (pad "32" thru_hole oval (at -2.54 -38.1 180) (size 1.7 1.7) (drill 1) (layers "*.Cu" "*.Mask") (remove_unused_layers no) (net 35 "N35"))
  (pad "33" thru_hole oval (at 0 -40.64 180) (size 1.7 1.7) (drill 1) (layers "*.Cu" "*.Mask") (remove_unused_layers no) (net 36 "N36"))
  (pad "34" thru_hole oval (at -2.54 -40.64 180) (size 1.7 1.7) (drill 1) (layers "*.Cu" "*.Mask") (remove_unused_layers no) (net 4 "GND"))
  (pad "35" thru_hole oval (at 0 -43.18 180) (size 1.7 1.7) (drill 1) (layers "*.Cu" "*.Mask") (remove_unused_layers no) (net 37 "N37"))
  (pad "36" thru_hole oval (at -2.54 -43.18 180) (size 1.7 1.7) (drill 1) (layers "*.Cu" "*.Mask") (remove_unused_layers no) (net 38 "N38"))
  (pad "37" thru_hole oval (at 0 -45.72 180) (size 1.7 1.7) (drill 1) (layers "*.Cu" "*.Mask") (remove_unused_layers no) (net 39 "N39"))
  (pad "38" thru_hole oval (at -2.54 -45.72 180) (size 1.7 1.7) (drill 1) (layers "*.Cu" "*.Mask") (remove_unused_layers no) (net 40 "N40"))
  (pad "39" thru_hole oval (at 0 -48.26 180) (size 1.7 1.7) (drill 1) (layers "*.Cu" "*.Mask") (remove_unused_layers no) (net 4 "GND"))
  (pad "40" thru_hole oval (at -2.54 -48.26 180) (size 1.7 1.7) (drill 1) (layers "*.Cu" "*.Mask") (remove_unused_layers no) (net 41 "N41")))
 (gr_rect (start 100.3 72) (end 126 95.6) (stroke (width 0.1) (type default)) (fill none) (layer "F.SilkS"))
 (gr_rect (start 128.8 71.88) (end 158.8 137.88) (stroke (width 0.1) (type default)) (fill none) (layer "F.SilkS"))
 (gr_rect (start 82 72) (end 98 94.8) (stroke (width 0.1) (type default)) (fill none) (layer "F.SilkS"))
 (gr_line (start 80.2 144.5) (end 80.2 64.7) (stroke (width 0.05) (type default)) (layer "Edge.Cuts"))
 (gr_line (start 160.2 64.3) (end 160.2 144.5) (stroke (width 0.05) (type default)) (layer "Edge.Cuts"))
 (gr_line (start 160.2 144.5) (end 80.2 144.5) (stroke (width 0.05) (type default)) (layer "Edge.Cuts"))
 (gr_line (start 80.2 64.7) (end 160.2 64.3) (stroke (width 0.05) (type default)) (layer "Edge.Cuts"))
 (segment (start 116.15 94.15) (end 116.15 74.6) (width 1.36703) (layer "F.Cu") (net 4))
 (segment (start 82 98) (end 83 99) (width 0.115469) (layer "F.Cu") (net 4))
 (segment (start 83.1 126) (end 99.1 142) (width 0.115469) (layer "F.Cu") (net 4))
 (segment (start 82.86 89.14) (end 82 90) (width 0.115469) (layer "F.Cu") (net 4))
 (segment (start 82 90) (end 82 98) (width 0.115469) (layer "F.Cu") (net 4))
 (segment (start 132.387735 142.105235) (end 136.894765 142.105235) (width 0.115469) (layer "F.Cu") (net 4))
 (segment (start 136.894765 142.105235) (end 137.992265 141.007735) (width 0.115469) (layer "F.Cu") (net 4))
 (segment (start 149.04203 129.04) (end 153.26 129.04) (width 0.115469) (layer "F.Cu") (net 4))
 (segment (start 116.15 70.61) (end 116.15 74.6) (width 2.03286) (layer "F.Cu") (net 4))
 (segment (start 131.38 141.0975) (end 132.387735 142.105235) (width 0.115469) (layer "F.Cu") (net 4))
 (segment (start 137.992265 141.007735) (end 137.992265 140.089765) (width 0.115469) (layer "F.Cu") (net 4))
 (segment (start 137.992265 140.089765) (end 149.04203 129.04) (width 0.115469) (layer "F.Cu") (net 4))
 (segment (start 84.6 89.14) (end 82.86 89.14) (width 0.115469) (layer "F.Cu") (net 4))
 (segment (start 126 104) (end 116.15 94.15) (width 1.36703) (layer "F.Cu") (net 4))
 (segment (start 114.54 69) (end 116.15 70.61) (width 2.03286) (layer "F.Cu") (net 4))
 (segment (start 99.1 142) (end 103 142) (width 0.115469) (layer "F.Cu") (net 4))
 (segment (start 114.368101 73.492265) (end 114.875836 74) (width 0.115469) (layer "F.Cu") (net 7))
 (segment (start 109.962265 73.492265) (end 107.771899 73.492265) (width 0.115469) (layer "F.Cu") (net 7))
 (segment (start 128 88) (end 132.68 83.32) (width 0.115469) (layer "F.Cu") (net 7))
 (segment (start 126 107) (end 128 107) (width 0.115469) (layer "F.Cu") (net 7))
 (segment (start 107.264164 75.735836) (end 98.94 84.06) (width 0.115469) (layer "F.Cu") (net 7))
 (segment (start 107.771899 73.492265) (end 107.264164 74) (width 0.115469) (layer "F.Cu") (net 7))
 (segment (start 132.68 83.32) (end 153.26 83.32) (width 0.115469) (layer "F.Cu") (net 7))
 (segment (start 128 107) (end 128 88) (width 0.115469) (layer "F.Cu") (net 7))
 (segment (start 114.875836 95.875836) (end 126 107) (width 0.115469) (layer "F.Cu") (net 7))
 (segment (start 112.177735 73.492265) (end 114.368101 73.492265) (width 0.115469) (layer "F.Cu") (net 7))
 (segment (start 114.875836 74) (end 114.875836 95.875836) (width 0.115469) (layer "F.Cu") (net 7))
 (segment (start 111.07 74.6) (end 112.177735 73.492265) (width 0.115469) (layer "F.Cu") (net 7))
 (segment (start 98.94 84.06) (end 84.6 84.06) (width 0.115469) (layer "F.Cu") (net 7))
 (segment (start 107.264164 74) (end 107.264164 75.735836) (width 0.115469) (layer "F.Cu") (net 7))
 (segment (start 111.07 74.6) (end 109.962265 73.492265) (width 0.115469) (layer "F.Cu") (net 7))
 (segment (start 124.057734 143.942266) (end 126 142) (width 0.115469) (layer "F.Cu") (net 1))
 (segment (start 88.942266 143.942266) (end 124.057734 143.942266) (width 0.115469) (layer "F.Cu") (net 1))
 (segment (start 137.335501 142.761999) (end 139 141.0975) (width 0.115469) (layer "F.Cu") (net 1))
 (segment (start 126 142) (end 126.761999 142.761999) (width 0.115469) (layer "F.Cu") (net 1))
 (segment (start 83.1 118.38) (end 81.992265 119.487735) (width 0.115469) (layer "F.Cu") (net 1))
 (segment (start 151.9025 141.0975) (end 158 135) (width 0.115469) (layer "F.Cu") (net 1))
 (segment (start 139 141.0975) (end 151.9025 141.0975) (width 0.115469) (layer "F.Cu") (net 1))
 (segment (start 126.761999 142.761999) (end 137.335501 142.761999) (width 0.115469) (layer "F.Cu") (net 1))
 (segment (start 81.992265 119.487735) (end 81.992265 136.992265) (width 0.115469) (layer "F.Cu") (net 1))
 (segment (start 158 82.98) (end 155.8 80.78) (width 0.115469) (layer "F.Cu") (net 1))
 (segment (start 158 135) (end 158 82.98) (width 0.115469) (layer "F.Cu") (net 1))
 (segment (start 81.992265 136.992265) (end 88.942266 143.942266) (width 0.115469) (layer "F.Cu") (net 1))
 (segment (start 136.46 133.14) (end 153.26 116.34) (width 0.115469) (layer "F.Cu") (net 12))
 (segment (start 136.46 141.0975) (end 136.46 133.14) (width 0.115469) (layer "F.Cu") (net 12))
 (segment (start 131 107) (end 131 89) (width 0.115469) (layer "F.Cu") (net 6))
 (segment (start 154.692265 84.427735) (end 153.26 85.86) (width 0.115469) (layer "F.Cu") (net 6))
 (segment (start 113.61 98.61) (end 125 110) (width 0.115469) (layer "F.Cu") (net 6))
 (segment (start 134.14 85.86) (end 153.26 85.86) (width 0.115469) (layer "F.Cu") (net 6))
 (segment (start 86.274164 67.725836) (end 142.421306 67.725836) (width 0.115469) (layer "F.Cu") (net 6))
 (segment (start 82.6 86.6) (end 82 86) (width 0.115469) (layer "F.Cu") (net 6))
 (segment (start 82 86) (end 82 72) (width 0.115469) (layer "F.Cu") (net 6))
 (segment (start 82 72) (end 86.274164 67.725836) (width 0.115469) (layer "F.Cu") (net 6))
 (segment (start 142.421306 67.725836) (end 154.692265 79.996795) (width 0.115469) (layer "F.Cu") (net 6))
 (segment (start 131 89) (end 134.14 85.86) (width 0.115469) (layer "F.Cu") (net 6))
 (segment (start 113.61 74.6) (end 113.61 98.61) (width 0.115469) (layer "F.Cu") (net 6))
 (segment (start 154.692265 79.996795) (end 154.692265 84.427735) (width 0.115469) (layer "F.Cu") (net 6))
 (segment (start 125 110) (end 128 110) (width 0.115469) (layer "F.Cu") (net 6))
 (segment (start 84.6 86.6) (end 82.6 86.6) (width 0.115469) (layer "F.Cu") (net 6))
 (segment (start 128 110) (end 131 107) (width 0.115469) (layer "F.Cu") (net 6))
 (segment (start 124 111) (end 143.36 111) (width 0.115469) (layer "F.Cu") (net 5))
 (segment (start 143.36 111) (end 153.26 101.1) (width 0.115469) (layer "F.Cu") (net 5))
 (segment (start 147.08 74.6) (end 153.26 80.78) (width 0.115469) (layer "F.Cu") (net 5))
 (segment (start 84.6 91.68) (end 84.6 93) (width 0.115469) (layer "F.Cu") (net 5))
 (segment (start 96.6 105) (end 97.6 106) (width 0.115469) (layer "F.Cu") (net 5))
 (segment (start 119 106) (end 124 111) (width 0.115469) (layer "F.Cu") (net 5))
 (segment (start 97.6 106) (end 119 106) (width 0.115469) (layer "F.Cu") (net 5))
 (segment (start 84.6 93) (end 96.6 105) (width 0.115469) (layer "F.Cu") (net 5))
 (segment (start 118.69 74.6) (end 147.08 74.6) (width 0.115469) (layer "F.Cu") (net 5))
 (segment (start 157 92.14) (end 155.8 90.94) (width 0.115469) (layer "F.Cu") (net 3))
 (segment (start 152.092265 114.907735) (end 156.258839 114.907735) (width 0.115469) (layer "F.Cu") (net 3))
 (segment (start 83.1 123.46) (end 85.56 121) (width 0.115469) (layer "F.Cu") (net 3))
 (segment (start 85.56 121) (end 146 121) (width 0.115469) (layer "F.Cu") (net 3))
 (segment (start 157 114.166574) (end 157 92.14) (width 0.115469) (layer "F.Cu") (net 3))
 (segment (start 146 121) (end 152.092265 114.907735) (width 0.115469) (layer "F.Cu") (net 3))
 (segment (start 156.258839 114.907735) (end 157 114.166574) (width 0.115469) (layer "F.Cu") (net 3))
 (segment (start 108.53 98.47) (end 103 104) (width 1.36703) (layer "F.Cu") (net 26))
 (segment (start 108.53 74.6) (end 108.53 98.47) (width 1.36703) (layer "F.Cu") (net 26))
 (segment (start 109.11714 69) (end 105.99 72.12714) (width 2.03286) (layer "F.Cu") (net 27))
 (segment (start 112 69) (end 109.11714 69) (width 2.03286) (layer "F.Cu") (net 27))
 (segment (start 105.99 72.12714) (end 105.99 74.6) (width 2.03286) (layer "F.Cu") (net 27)))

